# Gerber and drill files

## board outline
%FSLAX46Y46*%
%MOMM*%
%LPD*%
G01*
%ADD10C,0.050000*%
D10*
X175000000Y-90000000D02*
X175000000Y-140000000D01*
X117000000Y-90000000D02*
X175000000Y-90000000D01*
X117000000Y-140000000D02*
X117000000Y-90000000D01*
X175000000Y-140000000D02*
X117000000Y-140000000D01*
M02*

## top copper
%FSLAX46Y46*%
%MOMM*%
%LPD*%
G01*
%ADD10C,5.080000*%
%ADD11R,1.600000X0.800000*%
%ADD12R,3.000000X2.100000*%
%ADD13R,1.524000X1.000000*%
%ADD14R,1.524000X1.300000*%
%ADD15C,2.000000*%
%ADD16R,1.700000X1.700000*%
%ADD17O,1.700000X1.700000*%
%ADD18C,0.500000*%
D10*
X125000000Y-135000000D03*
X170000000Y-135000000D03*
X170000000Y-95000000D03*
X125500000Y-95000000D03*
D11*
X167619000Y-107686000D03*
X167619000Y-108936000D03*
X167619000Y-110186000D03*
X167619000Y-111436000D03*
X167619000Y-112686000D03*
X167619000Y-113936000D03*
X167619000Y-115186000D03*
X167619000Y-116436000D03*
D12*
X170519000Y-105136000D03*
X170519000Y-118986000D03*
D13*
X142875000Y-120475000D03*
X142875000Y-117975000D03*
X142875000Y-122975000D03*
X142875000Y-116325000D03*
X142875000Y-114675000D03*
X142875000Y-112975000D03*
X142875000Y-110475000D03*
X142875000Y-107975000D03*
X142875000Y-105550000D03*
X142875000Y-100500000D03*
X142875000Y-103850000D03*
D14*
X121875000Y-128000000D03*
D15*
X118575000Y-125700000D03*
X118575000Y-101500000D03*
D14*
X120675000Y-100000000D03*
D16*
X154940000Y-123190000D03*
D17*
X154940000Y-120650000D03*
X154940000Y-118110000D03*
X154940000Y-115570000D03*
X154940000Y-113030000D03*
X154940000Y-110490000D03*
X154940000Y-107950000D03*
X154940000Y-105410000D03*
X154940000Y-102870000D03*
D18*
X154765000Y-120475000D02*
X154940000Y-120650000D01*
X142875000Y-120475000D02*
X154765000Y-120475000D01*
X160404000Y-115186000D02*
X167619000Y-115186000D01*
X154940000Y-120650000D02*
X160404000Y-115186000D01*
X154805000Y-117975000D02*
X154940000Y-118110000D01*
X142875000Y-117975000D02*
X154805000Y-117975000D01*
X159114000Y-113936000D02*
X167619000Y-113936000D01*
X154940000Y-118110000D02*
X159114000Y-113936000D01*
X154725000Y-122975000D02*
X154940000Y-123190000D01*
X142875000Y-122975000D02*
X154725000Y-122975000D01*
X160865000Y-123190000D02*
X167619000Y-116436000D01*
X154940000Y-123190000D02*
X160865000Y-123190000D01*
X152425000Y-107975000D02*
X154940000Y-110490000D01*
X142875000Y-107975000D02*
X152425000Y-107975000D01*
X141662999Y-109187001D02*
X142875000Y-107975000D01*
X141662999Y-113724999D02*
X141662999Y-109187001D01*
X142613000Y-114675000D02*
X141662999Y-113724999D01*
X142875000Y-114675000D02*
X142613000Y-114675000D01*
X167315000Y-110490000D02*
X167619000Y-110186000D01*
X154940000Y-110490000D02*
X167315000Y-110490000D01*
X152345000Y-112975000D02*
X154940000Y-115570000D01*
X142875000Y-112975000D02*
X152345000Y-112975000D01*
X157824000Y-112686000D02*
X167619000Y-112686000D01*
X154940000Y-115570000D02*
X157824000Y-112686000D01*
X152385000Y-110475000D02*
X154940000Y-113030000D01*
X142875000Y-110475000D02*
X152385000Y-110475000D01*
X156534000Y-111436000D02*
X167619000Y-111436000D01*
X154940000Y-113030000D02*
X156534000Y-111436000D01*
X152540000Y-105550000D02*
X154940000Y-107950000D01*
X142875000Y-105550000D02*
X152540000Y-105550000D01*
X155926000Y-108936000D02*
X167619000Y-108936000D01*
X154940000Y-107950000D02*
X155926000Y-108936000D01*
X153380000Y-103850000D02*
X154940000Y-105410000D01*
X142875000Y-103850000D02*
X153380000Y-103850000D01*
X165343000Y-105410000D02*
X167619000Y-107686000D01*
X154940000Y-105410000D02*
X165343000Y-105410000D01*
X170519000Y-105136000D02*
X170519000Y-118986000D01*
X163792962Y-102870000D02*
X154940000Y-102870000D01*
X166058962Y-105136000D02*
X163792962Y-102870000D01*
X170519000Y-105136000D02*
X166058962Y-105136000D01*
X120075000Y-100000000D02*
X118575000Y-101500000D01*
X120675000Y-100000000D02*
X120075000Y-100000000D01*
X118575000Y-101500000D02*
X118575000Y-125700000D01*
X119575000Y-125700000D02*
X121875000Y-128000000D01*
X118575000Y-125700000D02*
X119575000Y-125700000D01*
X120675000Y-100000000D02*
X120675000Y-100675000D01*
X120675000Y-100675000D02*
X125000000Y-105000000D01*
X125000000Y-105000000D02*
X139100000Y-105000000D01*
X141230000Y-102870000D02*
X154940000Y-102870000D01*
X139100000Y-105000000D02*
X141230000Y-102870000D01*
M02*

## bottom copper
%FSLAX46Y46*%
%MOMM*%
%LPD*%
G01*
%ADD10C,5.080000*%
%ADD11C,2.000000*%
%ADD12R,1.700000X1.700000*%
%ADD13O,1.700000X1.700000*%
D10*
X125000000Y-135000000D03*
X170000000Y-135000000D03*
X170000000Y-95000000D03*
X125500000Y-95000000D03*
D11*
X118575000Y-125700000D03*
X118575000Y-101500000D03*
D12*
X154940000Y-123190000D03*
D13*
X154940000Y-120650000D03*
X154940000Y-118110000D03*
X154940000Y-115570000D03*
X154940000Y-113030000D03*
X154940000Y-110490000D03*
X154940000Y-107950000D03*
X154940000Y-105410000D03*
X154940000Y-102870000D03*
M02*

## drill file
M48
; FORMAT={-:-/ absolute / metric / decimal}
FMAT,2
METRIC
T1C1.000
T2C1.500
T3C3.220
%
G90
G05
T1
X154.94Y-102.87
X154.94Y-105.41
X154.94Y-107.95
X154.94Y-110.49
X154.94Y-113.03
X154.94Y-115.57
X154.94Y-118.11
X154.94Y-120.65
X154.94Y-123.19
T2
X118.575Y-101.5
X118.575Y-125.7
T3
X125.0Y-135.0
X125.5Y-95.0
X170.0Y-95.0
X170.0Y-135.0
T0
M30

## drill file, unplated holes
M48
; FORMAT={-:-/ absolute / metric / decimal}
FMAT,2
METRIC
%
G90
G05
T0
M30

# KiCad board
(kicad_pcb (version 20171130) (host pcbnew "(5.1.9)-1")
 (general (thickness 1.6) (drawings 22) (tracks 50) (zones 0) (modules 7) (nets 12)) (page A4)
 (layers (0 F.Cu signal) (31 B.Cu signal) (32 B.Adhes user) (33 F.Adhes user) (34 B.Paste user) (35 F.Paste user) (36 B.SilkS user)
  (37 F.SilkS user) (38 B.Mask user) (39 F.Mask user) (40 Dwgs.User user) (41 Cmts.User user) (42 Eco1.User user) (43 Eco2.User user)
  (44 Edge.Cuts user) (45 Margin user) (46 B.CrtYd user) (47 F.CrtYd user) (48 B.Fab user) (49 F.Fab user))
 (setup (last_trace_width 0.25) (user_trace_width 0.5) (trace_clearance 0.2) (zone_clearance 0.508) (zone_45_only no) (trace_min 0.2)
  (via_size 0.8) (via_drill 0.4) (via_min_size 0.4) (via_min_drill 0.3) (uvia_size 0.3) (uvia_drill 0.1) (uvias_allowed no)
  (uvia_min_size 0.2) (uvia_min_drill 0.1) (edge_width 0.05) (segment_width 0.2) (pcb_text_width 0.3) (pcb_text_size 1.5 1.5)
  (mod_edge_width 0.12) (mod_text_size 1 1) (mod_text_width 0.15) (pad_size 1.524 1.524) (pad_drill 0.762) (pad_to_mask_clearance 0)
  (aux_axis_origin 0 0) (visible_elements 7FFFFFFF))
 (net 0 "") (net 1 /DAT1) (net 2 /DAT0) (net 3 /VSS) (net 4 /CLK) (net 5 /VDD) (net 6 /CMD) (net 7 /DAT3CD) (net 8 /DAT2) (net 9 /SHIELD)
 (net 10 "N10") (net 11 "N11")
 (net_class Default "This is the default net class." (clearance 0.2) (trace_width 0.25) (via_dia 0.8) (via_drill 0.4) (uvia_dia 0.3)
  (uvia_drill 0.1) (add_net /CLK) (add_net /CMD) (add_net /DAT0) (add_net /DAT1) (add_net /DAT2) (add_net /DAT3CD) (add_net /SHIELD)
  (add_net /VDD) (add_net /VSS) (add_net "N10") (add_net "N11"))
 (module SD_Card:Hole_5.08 (layer F.Cu) (at 125 135)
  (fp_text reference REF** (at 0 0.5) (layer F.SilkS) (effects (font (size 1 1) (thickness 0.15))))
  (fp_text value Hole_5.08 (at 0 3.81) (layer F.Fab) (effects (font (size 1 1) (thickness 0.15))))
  (pad 1 thru_hole circle (at 0 0) (size 5.08 5.08) (drill 3.22) (layers *.Cu *.Mask)))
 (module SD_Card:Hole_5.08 (layer F.Cu) (at 170 135)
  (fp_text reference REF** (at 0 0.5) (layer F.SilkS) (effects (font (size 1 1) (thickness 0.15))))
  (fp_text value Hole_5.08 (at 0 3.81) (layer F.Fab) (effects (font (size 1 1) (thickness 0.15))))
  (pad 1 thru_hole circle (at 0 0) (size 5.08 5.08) (drill 3.22) (layers *.Cu *.Mask)))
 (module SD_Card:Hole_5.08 (layer F.Cu) (at 170 95)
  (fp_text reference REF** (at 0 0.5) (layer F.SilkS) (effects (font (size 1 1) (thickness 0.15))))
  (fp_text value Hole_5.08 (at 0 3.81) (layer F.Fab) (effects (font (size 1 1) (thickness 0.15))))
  (pad 1 thru_hole circle (at 0 0) (size 5.08 5.08) (drill 3.22) (layers *.Cu *.Mask)))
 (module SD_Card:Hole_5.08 (layer F.Cu) (at 125.5 95)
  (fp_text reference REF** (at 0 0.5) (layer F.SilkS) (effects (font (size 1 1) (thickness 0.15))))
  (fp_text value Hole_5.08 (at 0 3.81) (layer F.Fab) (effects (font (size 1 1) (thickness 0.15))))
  (pad 1 thru_hole circle (at 0 0) (size 5.08 5.08) (drill 3.22) (layers *.Cu *.Mask)))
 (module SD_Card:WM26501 (layer F.Cu) (at 170.667 112.258 270)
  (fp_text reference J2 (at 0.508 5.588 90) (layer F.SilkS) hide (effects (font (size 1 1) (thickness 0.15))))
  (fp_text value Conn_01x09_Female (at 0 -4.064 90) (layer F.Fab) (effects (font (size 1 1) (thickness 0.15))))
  (pad 8 smd rect (at -4.572 3.048 270) (size 0.8 1.6) (layers F.Cu F.Paste F.Mask) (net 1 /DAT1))
  (pad 7 smd rect (at -3.322 3.048 270) (size 0.8 1.6) (layers F.Cu F.Paste F.Mask) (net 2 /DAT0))
  (pad 6 smd rect (at -2.072 3.048 270) (size 0.8 1.6) (layers F.Cu F.Paste F.Mask) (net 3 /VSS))
  (pad 5 smd rect (at -0.822 3.048 270) (size 0.8 1.6) (layers F.Cu F.Paste F.Mask) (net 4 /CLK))
  (pad 4 smd rect (at 0.428 3.048 270) (size 0.8 1.6) (layers F.Cu F.Paste F.Mask) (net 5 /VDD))
  (pad 3 smd rect (at 1.678 3.048 270) (size 0.8 1.6) (layers F.Cu F.Paste F.Mask) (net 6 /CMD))
  (pad 2 smd rect (at 2.928 3.048 270) (size 0.8 1.6) (layers F.Cu F.Paste F.Mask) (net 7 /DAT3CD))
  (pad 1 smd rect (at 4.178 3.048 270) (size 0.8 1.6) (layers F.Cu F.Paste F.Mask) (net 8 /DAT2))
  (pad 9 smd rect (at -7.122 0.148 270) (size 2.1 3) (layers F.Cu F.Paste F.Mask) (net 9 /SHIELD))
  (pad 9 smd rect (at 6.728 0.148 270) (size 2.1 3) (layers F.Cu F.Paste F.Mask) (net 9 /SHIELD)))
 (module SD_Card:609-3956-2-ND (layer F.Cu) (at 142.875 110.475 270)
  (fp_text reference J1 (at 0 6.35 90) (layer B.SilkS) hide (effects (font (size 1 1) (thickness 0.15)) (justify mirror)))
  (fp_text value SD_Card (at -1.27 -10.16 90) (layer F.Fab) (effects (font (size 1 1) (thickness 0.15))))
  (pad 1 smd rect (at 10 0 270) (size 1 1.524) (layers F.Cu F.Paste F.Mask) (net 7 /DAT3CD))
  (pad 2 smd rect (at 7.5 0 270) (size 1 1.524) (layers F.Cu F.Paste F.Mask) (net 6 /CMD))
  (pad 9 smd rect (at 12.5 0 270) (size 1 1.524) (layers F.Cu F.Paste F.Mask) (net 8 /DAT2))
  (pad 10 smd rect (at 5.85 0 270) (size 1 1.524) (layers F.Cu F.Paste F.Mask) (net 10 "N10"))
  (pad 3 smd rect (at 4.2 0 270) (size 1 1.524) (layers F.Cu F.Paste F.Mask) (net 3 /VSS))
  (pad 4 smd rect (at 2.5 0 270) (size 1 1.524) (layers F.Cu F.Paste F.Mask) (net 5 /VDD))
  (pad 5 smd rect (at 0 0 270) (size 1 1.524) (layers F.Cu F.Paste F.Mask) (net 4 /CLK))
  (pad 6 smd rect (at -2.5 0 270) (size 1 1.524) (layers F.Cu F.Paste F.Mask) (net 3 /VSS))
  (pad 7 smd rect (at -4.925 0 270) (size 1 1.524) (layers F.Cu F.Paste F.Mask) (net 2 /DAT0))
  (pad 11 smd rect (at -9.975 0 270) (size 1 1.524) (layers F.Cu F.Paste F.Mask) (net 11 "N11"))
  (pad 8 smd rect (at -6.625 0 270) (size 1 1.524) (layers F.Cu F.Paste F.Mask) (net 1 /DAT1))
  (pad 12 smd rect (at 17.525 21 270) (size 1.3 1.524) (layers F.Cu F.Paste F.Mask) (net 9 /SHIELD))
  (pad 13 thru_hole circle (at 15.225 24.3 270) (size 2 2) (drill 1.5) (layers *.Cu *.Mask) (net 9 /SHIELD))
  (pad 13 thru_hole circle (at -8.975 24.3 270) (size 2 2) (drill 1.5) (layers *.Cu *.Mask) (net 9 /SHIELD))
  (pad 12 smd rect (at -10.475 22.2 270) (size 1.3 1.524) (layers F.Cu F.Paste F.Mask) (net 9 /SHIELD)))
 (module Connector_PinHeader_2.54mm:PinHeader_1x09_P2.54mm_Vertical (layer F.Cu) (at 154.94 123.19 180)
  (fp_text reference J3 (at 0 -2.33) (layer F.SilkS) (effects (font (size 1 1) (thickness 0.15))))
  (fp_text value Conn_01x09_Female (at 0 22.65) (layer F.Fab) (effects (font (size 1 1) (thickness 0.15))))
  (pad 1 thru_hole rect (at 0 0 180) (size 1.7 1.7) (drill 1) (layers *.Cu *.Mask) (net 8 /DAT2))
  (pad 2 thru_hole oval (at 0 2.54 180) (size 1.7 1.7) (drill 1) (layers *.Cu *.Mask) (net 7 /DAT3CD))
  (pad 3 thru_hole oval (at 0 5.08 180) (size 1.7 1.7) (drill 1) (layers *.Cu *.Mask) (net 6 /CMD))
  (pad 4 thru_hole oval (at 0 7.62 180) (size 1.7 1.7) (drill 1) (layers *.Cu *.Mask) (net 5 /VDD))
  (pad 5 thru_hole oval (at 0 10.16 180) (size 1.7 1.7) (drill 1) (layers *.Cu *.Mask) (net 4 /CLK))
  (pad 6 thru_hole oval (at 0 12.7 180) (size 1.7 1.7) (drill 1) (layers *.Cu *.Mask) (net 3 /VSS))
  (pad 7 thru_hole oval (at 0 15.24 180) (size 1.7 1.7) (drill 1) (layers *.Cu *.Mask) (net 2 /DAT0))
  (pad 8 thru_hole oval (at 0 17.78 180) (size 1.7 1.7) (drill 1) (layers *.Cu *.Mask) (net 1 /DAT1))
  (pad 9 thru_hole oval (at 0 20.32 180) (size 1.7 1.7) (drill 1) (layers *.Cu *.Mask) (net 9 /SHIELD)))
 (gr_line (start 175 90) (end 175 140) (layer Edge.Cuts) (width 0.05))
 (gr_line (start 117 90) (end 175 90) (layer Edge.Cuts) (width 0.05))
 (gr_line (start 117 140) (end 117 90) (layer Edge.Cuts) (width 0.05))
 (gr_line (start 175 140) (end 117 140) (layer Edge.Cuts) (width 0.05))
 (segment (start 154.765 120.475) (end 154.94 120.65) (width 0.5) (layer F.Cu) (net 7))
 (segment (start 142.875 120.475) (end 154.765 120.475) (width 0.5) (layer F.Cu) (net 7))
 (segment (start 160.404 115.186) (end 167.619 115.186) (width 0.5) (layer F.Cu) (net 7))
 (segment (start 154.94 120.65) (end 160.404 115.186) (width 0.5) (layer F.Cu) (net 7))
 (segment (start 154.805 117.975) (end 154.94 118.11) (width 0.5) (layer F.Cu) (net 6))
 (segment (start 142.875 117.975) (end 154.805 117.975) (width 0.5) (layer F.Cu) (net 6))
 (segment (start 159.114 113.936) (end 167.619 113.936) (width 0.5) (layer F.Cu) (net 6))
 (segment (start 154.94 118.11) (end 159.114 113.936) (width 0.5) (layer F.Cu) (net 6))
 (segment (start 154.725 122.975) (end 154.94 123.19) (width 0.5) (layer F.Cu) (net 8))
 (segment (start 142.875 122.975) (end 154.725 122.975) (width 0.5) (layer F.Cu) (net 8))
 (segment (start 160.865 123.19) (end 167.619 116.436) (width 0.5) (layer F.Cu) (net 8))
 (segment (start 154.94 123.19) (end 160.865 123.19) (width 0.5) (layer F.Cu) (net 8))
 (segment (start 152.425 107.975) (end 154.94 110.49) (width 0.5) (layer F.Cu) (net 3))
 (segment (start 142.875 107.975) (end 152.425 107.975) (width 0.5) (layer F.Cu) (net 3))
 (segment (start 141.662999 109.187001) (end 142.875 107.975) (width 0.5) (layer F.Cu) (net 3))
 (segment (start 141.662999 113.724999) (end 141.662999 109.187001) (width 0.5) (layer F.Cu) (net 3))
 (segment (start 142.613 114.675) (end 141.662999 113.724999) (width 0.5) (layer F.Cu) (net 3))
 (segment (start 142.875 114.675) (end 142.613 114.675) (width 0.5) (layer F.Cu) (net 3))
 (segment (start 167.315 110.49) (end 167.619 110.186) (width 0.5) (layer F.Cu) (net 3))
 (segment (start 154.94 110.49) (end 167.315 110.49) (width 0.5) (layer F.Cu) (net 3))
 (segment (start 152.345 112.975) (end 154.94 115.57) (width 0.5) (layer F.Cu) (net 5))
 (segment (start 142.875 112.975) (end 152.345 112.975) (width 0.5) (layer F.Cu) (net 5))
 (segment (start 157.824 112.686) (end 167.619 112.686) (width 0.5) (layer F.Cu) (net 5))
 (segment (start 154.94 115.57) (end 157.824 112.686) (width 0.5) (layer F.Cu) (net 5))
 (segment (start 152.385 110.475) (end 154.94 113.03) (width 0.5) (layer F.Cu) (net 4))
 (segment (start 142.875 110.475) (end 152.385 110.475) (width 0.5) (layer F.Cu) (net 4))
 (segment (start 156.534 111.436) (end 167.619 111.436) (width 0.5) (layer F.Cu) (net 4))
 (segment (start 154.94 113.03) (end 156.534 111.436) (width 0.5) (layer F.Cu) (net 4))
 (segment (start 152.54 105.55) (end 154.94 107.95) (width 0.5) (layer F.Cu) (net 2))
 (segment (start 142.875 105.55) (end 152.54 105.55) (width 0.5) (layer F.Cu) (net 2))
 (segment (start 155.926 108.936) (end 167.619 108.936) (width 0.5) (layer F.Cu) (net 2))
 (segment (start 154.94 107.95) (end 155.926 108.936) (width 0.5) (layer F.Cu) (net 2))
 (segment (start 153.38 103.85) (end 154.94 105.41) (width 0.5) (layer F.Cu) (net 1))
 (segment (start 142.875 103.85) (end 153.38 103.85) (width 0.5) (layer F.Cu) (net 1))
 (segment (start 165.343 105.41) (end 167.619 107.686) (width 0.5) (layer F.Cu) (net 1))
 (segment (start 154.94 105.41) (end 165.343 105.41) (width 0.5) (layer F.Cu) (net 1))
 (segment (start 170.519 105.136) (end 170.519 118.986) (width 0.5) (layer F.Cu) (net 9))
 (segment (start 163.792962 102.87) (end 154.94 102.87) (width 0.5) (layer F.Cu) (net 9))
 (segment (start 166.058962 105.136) (end 163.792962 102.87) (width 0.5) (layer F.Cu) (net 9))
 (segment (start 170.519 105.136) (end 166.058962 105.136) (width 0.5) (layer F.Cu) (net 9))
 (segment (start 120.075 100) (end 118.575 101.5) (width 0.5) (layer F.Cu) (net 9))
 (segment (start 120.675 100) (end 120.075 100) (width 0.5) (layer F.Cu) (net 9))
 (segment (start 118.575 101.5) (end 118.575 125.7) (width 0.5) (layer F.Cu) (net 9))
 (segment (start 119.575 125.7) (end 121.875 128) (width 0.5) (layer F.Cu) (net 9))
 (segment (start 118.575 125.7) (end 119.575 125.7) (width 0.5) (layer F.Cu) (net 9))
 (segment (start 120.675 100) (end 120.675 100.675) (width 0.5) (layer F.Cu) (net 9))
 (segment (start 120.675 100.675) (end 125 105) (width 0.5) (layer F.Cu) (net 9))
 (segment (start 125 105) (end 139.1 105) (width 0.5) (layer F.Cu) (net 9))
 (segment (start 141.23 102.87) (end 154.94 102.87) (width 0.5) (layer F.Cu) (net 9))
 (segment (start 139.1 105) (end 141.23 102.87) (width 0.5) (layer F.Cu) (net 9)))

